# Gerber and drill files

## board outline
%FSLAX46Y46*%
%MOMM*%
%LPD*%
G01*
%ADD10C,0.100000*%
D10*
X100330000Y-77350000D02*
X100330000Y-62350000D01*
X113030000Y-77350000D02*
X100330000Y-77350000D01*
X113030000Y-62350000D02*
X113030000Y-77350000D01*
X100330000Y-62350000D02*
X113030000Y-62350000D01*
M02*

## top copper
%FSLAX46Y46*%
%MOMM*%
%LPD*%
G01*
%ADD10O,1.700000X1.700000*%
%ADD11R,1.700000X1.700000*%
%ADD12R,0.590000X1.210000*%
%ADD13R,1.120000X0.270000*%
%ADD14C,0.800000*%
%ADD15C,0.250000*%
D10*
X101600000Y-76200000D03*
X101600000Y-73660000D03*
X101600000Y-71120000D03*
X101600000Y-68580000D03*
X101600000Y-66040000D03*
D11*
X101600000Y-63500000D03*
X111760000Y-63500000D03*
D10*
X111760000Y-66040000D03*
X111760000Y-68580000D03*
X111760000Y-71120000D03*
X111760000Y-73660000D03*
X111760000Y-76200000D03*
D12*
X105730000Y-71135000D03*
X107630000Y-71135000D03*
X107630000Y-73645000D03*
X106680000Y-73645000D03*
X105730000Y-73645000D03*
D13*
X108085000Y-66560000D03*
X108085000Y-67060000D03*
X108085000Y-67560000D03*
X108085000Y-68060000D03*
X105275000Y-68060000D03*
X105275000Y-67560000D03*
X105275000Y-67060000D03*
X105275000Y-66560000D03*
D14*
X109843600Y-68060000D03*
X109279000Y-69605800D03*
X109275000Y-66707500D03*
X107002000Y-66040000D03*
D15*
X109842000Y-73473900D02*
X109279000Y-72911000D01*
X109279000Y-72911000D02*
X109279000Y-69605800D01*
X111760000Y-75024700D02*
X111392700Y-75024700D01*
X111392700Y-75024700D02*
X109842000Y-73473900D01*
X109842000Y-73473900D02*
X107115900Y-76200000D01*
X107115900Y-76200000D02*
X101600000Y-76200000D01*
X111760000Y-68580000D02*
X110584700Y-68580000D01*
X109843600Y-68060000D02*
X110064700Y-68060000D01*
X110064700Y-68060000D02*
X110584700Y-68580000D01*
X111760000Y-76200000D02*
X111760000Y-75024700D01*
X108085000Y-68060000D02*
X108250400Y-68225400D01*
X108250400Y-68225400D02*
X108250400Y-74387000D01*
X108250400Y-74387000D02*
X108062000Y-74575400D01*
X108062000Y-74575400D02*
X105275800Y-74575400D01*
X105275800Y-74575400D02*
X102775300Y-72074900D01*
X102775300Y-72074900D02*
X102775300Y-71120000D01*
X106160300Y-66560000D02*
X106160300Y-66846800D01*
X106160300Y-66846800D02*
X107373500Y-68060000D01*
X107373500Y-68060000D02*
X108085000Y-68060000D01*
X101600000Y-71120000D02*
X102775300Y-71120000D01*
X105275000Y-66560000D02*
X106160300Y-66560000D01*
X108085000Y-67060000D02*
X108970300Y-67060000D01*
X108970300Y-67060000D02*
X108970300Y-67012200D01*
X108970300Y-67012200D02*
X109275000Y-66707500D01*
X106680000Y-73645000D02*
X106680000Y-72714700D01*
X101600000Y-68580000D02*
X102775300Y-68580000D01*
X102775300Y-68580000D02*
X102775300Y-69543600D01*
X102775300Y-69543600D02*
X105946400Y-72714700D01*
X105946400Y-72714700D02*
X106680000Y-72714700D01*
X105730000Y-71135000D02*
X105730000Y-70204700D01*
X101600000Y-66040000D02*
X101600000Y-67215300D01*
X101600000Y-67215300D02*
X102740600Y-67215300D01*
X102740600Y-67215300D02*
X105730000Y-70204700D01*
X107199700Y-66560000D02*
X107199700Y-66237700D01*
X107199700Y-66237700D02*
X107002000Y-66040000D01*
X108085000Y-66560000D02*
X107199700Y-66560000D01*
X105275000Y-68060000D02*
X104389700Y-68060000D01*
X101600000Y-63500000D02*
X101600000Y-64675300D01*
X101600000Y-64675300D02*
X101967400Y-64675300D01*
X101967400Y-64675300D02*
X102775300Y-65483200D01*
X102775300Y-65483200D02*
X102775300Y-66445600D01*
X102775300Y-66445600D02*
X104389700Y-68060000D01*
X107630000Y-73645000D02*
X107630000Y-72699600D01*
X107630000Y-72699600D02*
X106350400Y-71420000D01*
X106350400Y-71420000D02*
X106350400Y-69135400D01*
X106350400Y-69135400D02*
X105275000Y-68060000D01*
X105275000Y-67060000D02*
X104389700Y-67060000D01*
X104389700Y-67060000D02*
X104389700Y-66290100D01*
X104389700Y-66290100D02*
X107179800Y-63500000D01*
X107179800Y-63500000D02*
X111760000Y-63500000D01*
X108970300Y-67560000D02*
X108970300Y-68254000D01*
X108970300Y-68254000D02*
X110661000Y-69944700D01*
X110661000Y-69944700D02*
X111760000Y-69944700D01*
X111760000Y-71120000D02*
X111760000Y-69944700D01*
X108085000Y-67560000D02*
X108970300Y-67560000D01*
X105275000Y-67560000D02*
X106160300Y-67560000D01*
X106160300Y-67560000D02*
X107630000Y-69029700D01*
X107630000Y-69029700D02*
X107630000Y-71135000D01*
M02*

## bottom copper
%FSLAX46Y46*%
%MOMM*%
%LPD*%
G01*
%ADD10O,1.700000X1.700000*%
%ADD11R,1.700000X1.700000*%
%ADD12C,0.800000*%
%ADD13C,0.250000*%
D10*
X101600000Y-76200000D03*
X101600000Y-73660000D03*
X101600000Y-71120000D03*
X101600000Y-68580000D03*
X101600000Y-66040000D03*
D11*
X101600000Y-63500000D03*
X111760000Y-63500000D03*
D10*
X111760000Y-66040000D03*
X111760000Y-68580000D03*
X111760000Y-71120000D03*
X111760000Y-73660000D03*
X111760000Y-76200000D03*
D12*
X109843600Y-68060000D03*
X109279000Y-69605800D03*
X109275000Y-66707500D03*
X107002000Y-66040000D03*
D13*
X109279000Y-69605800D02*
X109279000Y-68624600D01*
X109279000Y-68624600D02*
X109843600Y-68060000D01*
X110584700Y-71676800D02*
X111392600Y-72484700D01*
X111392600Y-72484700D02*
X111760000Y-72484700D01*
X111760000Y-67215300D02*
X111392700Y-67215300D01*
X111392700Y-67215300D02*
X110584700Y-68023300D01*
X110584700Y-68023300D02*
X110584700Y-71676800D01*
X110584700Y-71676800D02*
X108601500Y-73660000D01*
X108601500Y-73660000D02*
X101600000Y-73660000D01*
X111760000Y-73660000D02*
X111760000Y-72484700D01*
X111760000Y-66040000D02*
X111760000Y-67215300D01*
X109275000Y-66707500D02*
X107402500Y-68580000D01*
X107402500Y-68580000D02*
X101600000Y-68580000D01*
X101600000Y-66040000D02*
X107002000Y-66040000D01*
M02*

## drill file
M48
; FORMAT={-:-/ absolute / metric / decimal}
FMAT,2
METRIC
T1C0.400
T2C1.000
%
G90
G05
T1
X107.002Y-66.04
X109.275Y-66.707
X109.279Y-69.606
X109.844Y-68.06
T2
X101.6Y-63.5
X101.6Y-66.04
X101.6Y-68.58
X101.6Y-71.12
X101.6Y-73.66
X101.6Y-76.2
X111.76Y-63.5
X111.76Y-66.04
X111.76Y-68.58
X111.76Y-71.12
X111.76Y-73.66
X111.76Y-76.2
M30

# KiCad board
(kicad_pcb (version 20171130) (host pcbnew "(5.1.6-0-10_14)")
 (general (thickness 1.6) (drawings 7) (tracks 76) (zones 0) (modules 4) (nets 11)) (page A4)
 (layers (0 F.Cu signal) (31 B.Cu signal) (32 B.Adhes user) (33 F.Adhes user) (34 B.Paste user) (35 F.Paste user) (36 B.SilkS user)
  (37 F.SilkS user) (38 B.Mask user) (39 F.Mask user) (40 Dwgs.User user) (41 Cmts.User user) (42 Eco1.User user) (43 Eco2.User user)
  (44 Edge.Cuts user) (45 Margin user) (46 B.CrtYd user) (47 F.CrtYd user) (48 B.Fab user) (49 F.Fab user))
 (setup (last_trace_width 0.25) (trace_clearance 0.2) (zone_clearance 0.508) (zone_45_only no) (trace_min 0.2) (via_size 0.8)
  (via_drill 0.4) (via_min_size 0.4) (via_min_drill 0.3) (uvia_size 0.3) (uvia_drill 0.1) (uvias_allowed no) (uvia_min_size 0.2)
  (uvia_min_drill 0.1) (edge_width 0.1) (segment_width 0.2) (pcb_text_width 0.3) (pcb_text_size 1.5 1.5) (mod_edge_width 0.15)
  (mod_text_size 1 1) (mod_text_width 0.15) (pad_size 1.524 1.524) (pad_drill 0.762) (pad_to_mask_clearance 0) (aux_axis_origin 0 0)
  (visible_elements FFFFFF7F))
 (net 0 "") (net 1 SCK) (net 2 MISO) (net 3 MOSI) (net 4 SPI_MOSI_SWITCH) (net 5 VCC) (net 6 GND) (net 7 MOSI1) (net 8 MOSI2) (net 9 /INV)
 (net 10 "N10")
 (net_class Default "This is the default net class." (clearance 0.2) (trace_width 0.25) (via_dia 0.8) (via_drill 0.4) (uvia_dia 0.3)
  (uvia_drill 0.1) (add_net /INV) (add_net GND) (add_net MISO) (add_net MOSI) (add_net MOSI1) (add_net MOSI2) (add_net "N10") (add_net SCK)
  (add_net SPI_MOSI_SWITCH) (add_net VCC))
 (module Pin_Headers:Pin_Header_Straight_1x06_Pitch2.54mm (layer F.Cu) (at 101.6 63.5)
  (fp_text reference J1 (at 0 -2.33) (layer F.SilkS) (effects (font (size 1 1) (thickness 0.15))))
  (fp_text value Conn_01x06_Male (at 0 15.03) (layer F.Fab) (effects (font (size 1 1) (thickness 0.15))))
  (pad 6 thru_hole oval (at 0 12.7) (size 1.7 1.7) (drill 1) (layers *.Cu *.Mask) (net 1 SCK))
  (pad 5 thru_hole oval (at 0 10.16) (size 1.7 1.7) (drill 1) (layers *.Cu *.Mask) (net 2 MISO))
  (pad 4 thru_hole oval (at 0 7.62) (size 1.7 1.7) (drill 1) (layers *.Cu *.Mask) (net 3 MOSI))
  (pad 3 thru_hole oval (at 0 5.08) (size 1.7 1.7) (drill 1) (layers *.Cu *.Mask) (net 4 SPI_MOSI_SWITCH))
  (pad 2 thru_hole oval (at 0 2.54) (size 1.7 1.7) (drill 1) (layers *.Cu *.Mask) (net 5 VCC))
  (pad 1 thru_hole rect (at 0 0) (size 1.7 1.7) (drill 1) (layers *.Cu *.Mask) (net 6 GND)))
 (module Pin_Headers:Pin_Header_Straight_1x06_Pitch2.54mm (layer F.Cu) (at 111.76 63.5)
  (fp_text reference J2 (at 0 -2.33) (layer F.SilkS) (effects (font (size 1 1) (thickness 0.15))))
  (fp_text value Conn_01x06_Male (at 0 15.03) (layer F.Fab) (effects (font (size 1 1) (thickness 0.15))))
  (pad 1 thru_hole rect (at 0 0) (size 1.7 1.7) (drill 1) (layers *.Cu *.Mask) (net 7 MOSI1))
  (pad 2 thru_hole oval (at 0 2.54) (size 1.7 1.7) (drill 1) (layers *.Cu *.Mask) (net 2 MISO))
  (pad 3 thru_hole oval (at 0 5.08) (size 1.7 1.7) (drill 1) (layers *.Cu *.Mask) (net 1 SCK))
  (pad 4 thru_hole oval (at 0 7.62) (size 1.7 1.7) (drill 1) (layers *.Cu *.Mask) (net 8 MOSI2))
  (pad 5 thru_hole oval (at 0 10.16) (size 1.7 1.7) (drill 1) (layers *.Cu *.Mask) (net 2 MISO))
  (pad 6 thru_hole oval (at 0 12.7) (size 1.7 1.7) (drill 1) (layers *.Cu *.Mask) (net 1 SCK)))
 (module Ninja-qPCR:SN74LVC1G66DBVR (layer F.Cu) (at 106.68 72.39 90)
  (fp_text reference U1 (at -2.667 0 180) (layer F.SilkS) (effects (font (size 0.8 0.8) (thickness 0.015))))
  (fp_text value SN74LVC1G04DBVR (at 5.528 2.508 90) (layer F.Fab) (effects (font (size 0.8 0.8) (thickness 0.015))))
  (pad 5 smd rect (at 1.255 -0.95 90) (size 1.21 0.59) (layers F.Cu F.Paste F.Mask) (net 5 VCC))
  (pad 4 smd rect (at 1.255 0.95 90) (size 1.21 0.59) (layers F.Cu F.Paste F.Mask) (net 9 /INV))
  (pad 3 smd rect (at -1.255 0.95 90) (size 1.21 0.59) (layers F.Cu F.Paste F.Mask) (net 6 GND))
  (pad 2 smd rect (at -1.255 0 90) (size 1.21 0.59) (layers F.Cu F.Paste F.Mask) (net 4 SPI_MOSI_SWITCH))
  (pad 1 smd rect (at -1.255 -0.95 90) (size 1.21 0.59) (layers F.Cu F.Paste F.Mask) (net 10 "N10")))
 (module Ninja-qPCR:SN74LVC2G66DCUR (layer F.Cu) (at 106.68 67.31)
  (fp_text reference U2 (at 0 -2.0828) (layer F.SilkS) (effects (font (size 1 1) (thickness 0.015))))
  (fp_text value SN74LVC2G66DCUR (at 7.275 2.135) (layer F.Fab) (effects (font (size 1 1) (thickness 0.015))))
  (pad 8 smd rect (at 1.405 -0.75) (size 1.12 0.27) (layers F.Cu F.Paste F.Mask) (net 5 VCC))
  (pad 7 smd rect (at 1.405 -0.25) (size 1.12 0.27) (layers F.Cu F.Paste F.Mask) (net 4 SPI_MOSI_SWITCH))
  (pad 6 smd rect (at 1.405 0.25) (size 1.12 0.27) (layers F.Cu F.Paste F.Mask) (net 8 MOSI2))
  (pad 5 smd rect (at 1.405 0.75) (size 1.12 0.27) (layers F.Cu F.Paste F.Mask) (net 3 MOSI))
  (pad 4 smd rect (at -1.405 0.75) (size 1.12 0.27) (layers F.Cu F.Paste F.Mask) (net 6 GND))
  (pad 3 smd rect (at -1.405 0.25) (size 1.12 0.27) (layers F.Cu F.Paste F.Mask) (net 9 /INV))
  (pad 2 smd rect (at -1.405 -0.25) (size 1.12 0.27) (layers F.Cu F.Paste F.Mask) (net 7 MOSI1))
  (pad 1 smd rect (at -1.405 -0.75) (size 1.12 0.27) (layers F.Cu F.Paste F.Mask) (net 3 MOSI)))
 (gr_line (start 100.33 77.35) (end 100.33 62.35) (layer Edge.Cuts) (width 0.1))
 (gr_line (start 113.03 77.35) (end 100.33 77.35) (layer Edge.Cuts) (width 0.1))
 (gr_line (start 113.03 62.35) (end 113.03 77.35) (layer Edge.Cuts) (width 0.1))
 (gr_line (start 100.33 62.35) (end 113.03 62.35) (layer Edge.Cuts) (width 0.1))
 (segment (start 109.842 73.4739) (end 109.279 72.911) (width 0.25) (layer F.Cu) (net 1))
 (segment (start 109.279 72.911) (end 109.279 69.6058) (width 0.25) (layer F.Cu) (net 1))
 (segment (start 111.76 75.0247) (end 111.3927 75.0247) (width 0.25) (layer F.Cu) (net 1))
 (segment (start 111.3927 75.0247) (end 109.842 73.4739) (width 0.25) (layer F.Cu) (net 1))
 (segment (start 109.842 73.4739) (end 107.1159 76.2) (width 0.25) (layer F.Cu) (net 1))
 (segment (start 107.1159 76.2) (end 101.6 76.2) (width 0.25) (layer F.Cu) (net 1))
 (segment (start 111.76 68.58) (end 110.5847 68.58) (width 0.25) (layer F.Cu) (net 1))
 (segment (start 109.8436 68.06) (end 110.0647 68.06) (width 0.25) (layer F.Cu) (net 1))
 (segment (start 110.0647 68.06) (end 110.5847 68.58) (width 0.25) (layer F.Cu) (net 1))
 (segment (start 109.279 69.6058) (end 109.279 68.6246) (width 0.25) (layer B.Cu) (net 1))
 (segment (start 109.279 68.6246) (end 109.8436 68.06) (width 0.25) (layer B.Cu) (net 1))
 (segment (start 111.76 76.2) (end 111.76 75.0247) (width 0.25) (layer F.Cu) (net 1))
 (via (at 109.8436 68.06) (size 0.8) (layers F.Cu B.Cu) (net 1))
 (via (at 109.279 69.6058) (size 0.8) (layers F.Cu B.Cu) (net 1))
 (segment (start 110.5847 71.6768) (end 111.3926 72.4847) (width 0.25) (layer B.Cu) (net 2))
 (segment (start 111.3926 72.4847) (end 111.76 72.4847) (width 0.25) (layer B.Cu) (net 2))
 (segment (start 111.76 67.2153) (end 111.3927 67.2153) (width 0.25) (layer B.Cu) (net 2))
 (segment (start 111.3927 67.2153) (end 110.5847 68.0233) (width 0.25) (layer B.Cu) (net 2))
 (segment (start 110.5847 68.0233) (end 110.5847 71.6768) (width 0.25) (layer B.Cu) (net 2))
 (segment (start 110.5847 71.6768) (end 108.6015 73.66) (width 0.25) (layer B.Cu) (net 2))
 (segment (start 108.6015 73.66) (end 101.6 73.66) (width 0.25) (layer B.Cu) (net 2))
 (segment (start 111.76 73.66) (end 111.76 72.4847) (width 0.25) (layer B.Cu) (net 2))
 (segment (start 111.76 66.04) (end 111.76 67.2153) (width 0.25) (layer B.Cu) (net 2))
 (segment (start 108.085 68.06) (end 108.2504 68.2254) (width 0.25) (layer F.Cu) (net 3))
 (segment (start 108.2504 68.2254) (end 108.2504 74.387) (width 0.25) (layer F.Cu) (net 3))
 (segment (start 108.2504 74.387) (end 108.062 74.5754) (width 0.25) (layer F.Cu) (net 3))
 (segment (start 108.062 74.5754) (end 105.2758 74.5754) (width 0.25) (layer F.Cu) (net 3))
 (segment (start 105.2758 74.5754) (end 102.7753 72.0749) (width 0.25) (layer F.Cu) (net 3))
 (segment (start 102.7753 72.0749) (end 102.7753 71.12) (width 0.25) (layer F.Cu) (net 3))
 (segment (start 106.1603 66.56) (end 106.1603 66.8468) (width 0.25) (layer F.Cu) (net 3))
 (segment (start 106.1603 66.8468) (end 107.3735 68.06) (width 0.25) (layer F.Cu) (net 3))
 (segment (start 107.3735 68.06) (end 108.085 68.06) (width 0.25) (layer F.Cu) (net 3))
 (segment (start 101.6 71.12) (end 102.7753 71.12) (width 0.25) (layer F.Cu) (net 3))
 (segment (start 105.275 66.56) (end 106.1603 66.56) (width 0.25) (layer F.Cu) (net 3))
 (segment (start 108.085 67.06) (end 108.9703 67.06) (width 0.25) (layer F.Cu) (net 4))
 (segment (start 109.275 66.7075) (end 107.4025 68.58) (width 0.25) (layer B.Cu) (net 4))
 (segment (start 107.4025 68.58) (end 101.6 68.58) (width 0.25) (layer B.Cu) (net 4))
 (segment (start 108.9703 67.06) (end 108.9703 67.0122) (width 0.25) (layer F.Cu) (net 4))
 (segment (start 108.9703 67.0122) (end 109.275 66.7075) (width 0.25) (layer F.Cu) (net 4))
 (segment (start 106.68 73.645) (end 106.68 72.7147) (width 0.25) (layer F.Cu) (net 4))
 (segment (start 101.6 68.58) (end 102.7753 68.58) (width 0.25) (layer F.Cu) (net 4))
 (segment (start 102.7753 68.58) (end 102.7753 69.5436) (width 0.25) (layer F.Cu) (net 4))
 (segment (start 102.7753 69.5436) (end 105.9464 72.7147) (width 0.25) (layer F.Cu) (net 4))
 (segment (start 105.9464 72.7147) (end 106.68 72.7147) (width 0.25) (layer F.Cu) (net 4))
 (via (at 109.275 66.7075) (size 0.8) (layers F.Cu B.Cu) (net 4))
 (segment (start 105.73 71.135) (end 105.73 70.2047) (width 0.25) (layer F.Cu) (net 5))
 (segment (start 101.6 66.04) (end 101.6 67.2153) (width 0.25) (layer F.Cu) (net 5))
 (segment (start 101.6 67.2153) (end 102.7406 67.2153) (width 0.25) (layer F.Cu) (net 5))
 (segment (start 102.7406 67.2153) (end 105.73 70.2047) (width 0.25) (layer F.Cu) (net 5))
 (segment (start 107.1997 66.56) (end 107.1997 66.2377) (width 0.25) (layer F.Cu) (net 5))
 (segment (start 107.1997 66.2377) (end 107.002 66.04) (width 0.25) (layer F.Cu) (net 5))
 (segment (start 101.6 66.04) (end 107.002 66.04) (width 0.25) (layer B.Cu) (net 5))
 (segment (start 108.085 66.56) (end 107.1997 66.56) (width 0.25) (layer F.Cu) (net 5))
 (via (at 107.002 66.04) (size 0.8) (layers F.Cu B.Cu) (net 5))
 (segment (start 105.275 68.06) (end 104.3897 68.06) (width 0.25) (layer F.Cu) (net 6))
 (segment (start 101.6 63.5) (end 101.6 64.6753) (width 0.25) (layer F.Cu) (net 6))
 (segment (start 101.6 64.6753) (end 101.9674 64.6753) (width 0.25) (layer F.Cu) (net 6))
 (segment (start 101.9674 64.6753) (end 102.7753 65.4832) (width 0.25) (layer F.Cu) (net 6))
 (segment (start 102.7753 65.4832) (end 102.7753 66.4456) (width 0.25) (layer F.Cu) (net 6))
 (segment (start 102.7753 66.4456) (end 104.3897 68.06) (width 0.25) (layer F.Cu) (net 6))
 (segment (start 107.63 73.645) (end 107.63 72.6996) (width 0.25) (layer F.Cu) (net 6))
 (segment (start 107.63 72.6996) (end 106.3504 71.42) (width 0.25) (layer F.Cu) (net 6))
 (segment (start 106.3504 71.42) (end 106.3504 69.1354) (width 0.25) (layer F.Cu) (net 6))
 (segment (start 106.3504 69.1354) (end 105.275 68.06) (width 0.25) (layer F.Cu) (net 6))
 (segment (start 105.275 67.06) (end 104.3897 67.06) (width 0.25) (layer F.Cu) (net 7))
 (segment (start 104.3897 67.06) (end 104.3897 66.2901) (width 0.25) (layer F.Cu) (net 7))
 (segment (start 104.3897 66.2901) (end 107.1798 63.5) (width 0.25) (layer F.Cu) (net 7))
 (segment (start 107.1798 63.5) (end 111.76 63.5) (width 0.25) (layer F.Cu) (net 7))
 (segment (start 108.9703 67.56) (end 108.9703 68.254) (width 0.25) (layer F.Cu) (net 8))
 (segment (start 108.9703 68.254) (end 110.661 69.9447) (width 0.25) (layer F.Cu) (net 8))
 (segment (start 110.661 69.9447) (end 111.76 69.9447) (width 0.25) (layer F.Cu) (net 8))
 (segment (start 111.76 71.12) (end 111.76 69.9447) (width 0.25) (layer F.Cu) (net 8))
 (segment (start 108.085 67.56) (end 108.9703 67.56) (width 0.25) (layer F.Cu) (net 8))
 (segment (start 105.275 67.56) (end 106.1603 67.56) (width 0.25) (layer F.Cu) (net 9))
 (segment (start 106.1603 67.56) (end 107.63 69.0297) (width 0.25) (layer F.Cu) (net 9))
 (segment (start 107.63 69.0297) (end 107.63 71.135) (width 0.25) (layer F.Cu) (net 9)))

